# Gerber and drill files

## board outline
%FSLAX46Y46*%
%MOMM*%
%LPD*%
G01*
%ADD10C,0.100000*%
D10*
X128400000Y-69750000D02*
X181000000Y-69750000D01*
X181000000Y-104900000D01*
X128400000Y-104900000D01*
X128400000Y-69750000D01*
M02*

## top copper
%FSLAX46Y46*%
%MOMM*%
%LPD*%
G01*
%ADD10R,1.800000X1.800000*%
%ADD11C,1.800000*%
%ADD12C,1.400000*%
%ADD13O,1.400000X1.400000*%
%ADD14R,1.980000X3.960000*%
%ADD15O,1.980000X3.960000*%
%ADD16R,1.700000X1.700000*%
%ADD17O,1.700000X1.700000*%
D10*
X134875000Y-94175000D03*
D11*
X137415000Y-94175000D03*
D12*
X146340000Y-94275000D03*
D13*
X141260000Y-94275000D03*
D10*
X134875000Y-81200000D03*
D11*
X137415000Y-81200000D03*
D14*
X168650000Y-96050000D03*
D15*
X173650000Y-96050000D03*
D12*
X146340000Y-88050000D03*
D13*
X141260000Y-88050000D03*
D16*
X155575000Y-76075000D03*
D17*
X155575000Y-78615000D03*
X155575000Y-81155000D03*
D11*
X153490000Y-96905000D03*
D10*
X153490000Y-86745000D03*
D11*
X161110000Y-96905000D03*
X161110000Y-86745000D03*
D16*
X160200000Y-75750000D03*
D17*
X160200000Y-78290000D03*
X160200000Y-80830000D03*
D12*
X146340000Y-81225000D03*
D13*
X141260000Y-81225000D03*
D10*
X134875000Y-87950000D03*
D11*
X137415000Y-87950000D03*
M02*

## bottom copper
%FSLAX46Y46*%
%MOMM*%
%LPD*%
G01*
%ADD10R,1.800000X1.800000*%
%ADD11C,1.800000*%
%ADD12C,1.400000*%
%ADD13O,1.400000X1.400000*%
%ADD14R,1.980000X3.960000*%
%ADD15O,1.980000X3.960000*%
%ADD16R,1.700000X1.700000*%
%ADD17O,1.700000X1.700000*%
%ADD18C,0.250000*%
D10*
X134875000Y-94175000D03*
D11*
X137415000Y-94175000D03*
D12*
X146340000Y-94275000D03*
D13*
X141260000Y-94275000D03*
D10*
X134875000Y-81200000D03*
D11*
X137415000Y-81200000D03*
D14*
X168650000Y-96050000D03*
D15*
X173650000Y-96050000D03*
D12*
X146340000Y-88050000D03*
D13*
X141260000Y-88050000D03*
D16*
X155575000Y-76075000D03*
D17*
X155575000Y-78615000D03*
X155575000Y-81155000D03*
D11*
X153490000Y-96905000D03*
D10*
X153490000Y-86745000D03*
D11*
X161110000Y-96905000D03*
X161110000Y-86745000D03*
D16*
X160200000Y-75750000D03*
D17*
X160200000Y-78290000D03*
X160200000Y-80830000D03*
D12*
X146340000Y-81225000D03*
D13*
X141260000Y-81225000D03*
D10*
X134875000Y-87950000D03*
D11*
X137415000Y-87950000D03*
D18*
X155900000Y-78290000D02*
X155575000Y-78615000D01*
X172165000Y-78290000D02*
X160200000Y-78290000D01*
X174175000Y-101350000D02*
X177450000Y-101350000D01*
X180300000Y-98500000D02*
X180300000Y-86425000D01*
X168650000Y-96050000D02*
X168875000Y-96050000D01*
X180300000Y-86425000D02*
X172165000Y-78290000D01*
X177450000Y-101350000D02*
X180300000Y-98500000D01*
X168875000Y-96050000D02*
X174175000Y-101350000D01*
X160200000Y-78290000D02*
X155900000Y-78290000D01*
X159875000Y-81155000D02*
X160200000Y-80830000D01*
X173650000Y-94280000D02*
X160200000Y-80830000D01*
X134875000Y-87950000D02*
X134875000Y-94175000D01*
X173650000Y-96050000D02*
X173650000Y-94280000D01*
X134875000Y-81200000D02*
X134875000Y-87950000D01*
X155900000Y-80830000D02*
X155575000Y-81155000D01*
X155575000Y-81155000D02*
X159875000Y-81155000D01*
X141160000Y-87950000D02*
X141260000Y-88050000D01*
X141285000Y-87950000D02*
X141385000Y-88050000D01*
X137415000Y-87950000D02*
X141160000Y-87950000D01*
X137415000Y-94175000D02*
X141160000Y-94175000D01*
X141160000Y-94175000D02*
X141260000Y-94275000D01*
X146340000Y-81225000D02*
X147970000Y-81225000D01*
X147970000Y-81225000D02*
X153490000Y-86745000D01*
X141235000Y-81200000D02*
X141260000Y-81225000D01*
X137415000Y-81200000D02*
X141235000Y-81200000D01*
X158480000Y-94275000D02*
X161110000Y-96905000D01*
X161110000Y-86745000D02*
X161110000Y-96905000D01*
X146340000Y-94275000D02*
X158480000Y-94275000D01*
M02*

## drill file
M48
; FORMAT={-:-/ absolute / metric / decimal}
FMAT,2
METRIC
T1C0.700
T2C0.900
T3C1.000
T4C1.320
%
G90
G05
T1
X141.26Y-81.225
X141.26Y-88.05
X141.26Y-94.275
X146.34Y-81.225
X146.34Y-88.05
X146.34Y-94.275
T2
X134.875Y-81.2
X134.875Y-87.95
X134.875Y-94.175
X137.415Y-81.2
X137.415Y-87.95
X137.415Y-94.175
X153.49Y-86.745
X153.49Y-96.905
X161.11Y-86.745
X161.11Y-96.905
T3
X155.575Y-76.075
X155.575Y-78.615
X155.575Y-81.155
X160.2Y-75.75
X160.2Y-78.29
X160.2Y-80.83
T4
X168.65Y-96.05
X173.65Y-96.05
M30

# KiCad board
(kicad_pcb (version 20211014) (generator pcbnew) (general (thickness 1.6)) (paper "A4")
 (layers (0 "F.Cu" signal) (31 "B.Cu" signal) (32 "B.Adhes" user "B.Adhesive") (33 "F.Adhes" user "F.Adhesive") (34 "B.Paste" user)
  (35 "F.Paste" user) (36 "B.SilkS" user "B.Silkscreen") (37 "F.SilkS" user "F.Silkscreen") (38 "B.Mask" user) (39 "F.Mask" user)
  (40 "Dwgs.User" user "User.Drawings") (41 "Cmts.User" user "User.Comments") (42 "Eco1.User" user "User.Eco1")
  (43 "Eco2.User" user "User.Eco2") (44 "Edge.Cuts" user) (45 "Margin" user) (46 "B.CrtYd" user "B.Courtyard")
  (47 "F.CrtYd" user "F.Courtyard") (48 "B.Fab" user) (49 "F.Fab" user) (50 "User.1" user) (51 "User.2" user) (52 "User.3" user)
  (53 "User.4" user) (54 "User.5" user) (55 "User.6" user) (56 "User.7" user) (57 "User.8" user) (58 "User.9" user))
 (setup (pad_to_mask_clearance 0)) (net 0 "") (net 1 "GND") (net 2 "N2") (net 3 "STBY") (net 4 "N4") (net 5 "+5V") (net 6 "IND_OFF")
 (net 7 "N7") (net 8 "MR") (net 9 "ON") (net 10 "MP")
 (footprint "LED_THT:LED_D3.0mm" (layer "F.Cu") (at 134.875 94.175)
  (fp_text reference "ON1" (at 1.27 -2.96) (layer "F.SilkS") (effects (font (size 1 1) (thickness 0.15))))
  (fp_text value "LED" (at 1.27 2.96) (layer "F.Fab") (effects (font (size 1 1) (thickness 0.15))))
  (pad "1" thru_hole rect (at 0 0) (size 1.8 1.8) (drill 0.9) (layers *.Cu *.Mask) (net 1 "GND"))
  (pad "2" thru_hole circle (at 2.54 0) (size 1.8 1.8) (drill 0.9) (layers *.Cu *.Mask) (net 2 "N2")))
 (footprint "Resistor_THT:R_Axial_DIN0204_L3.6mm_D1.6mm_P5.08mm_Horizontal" (layer "F.Cu") (at 146.34 94.275 180)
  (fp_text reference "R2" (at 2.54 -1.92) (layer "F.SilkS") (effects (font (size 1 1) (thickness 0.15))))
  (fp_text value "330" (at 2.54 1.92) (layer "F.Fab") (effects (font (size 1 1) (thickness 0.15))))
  (pad "1" thru_hole circle (at 0 0 180) (size 1.4 1.4) (drill 0.7) (layers *.Cu *.Mask) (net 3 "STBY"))
  (pad "2" thru_hole oval (at 5.08 0 180) (size 1.4 1.4) (drill 0.7) (layers *.Cu *.Mask) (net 2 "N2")))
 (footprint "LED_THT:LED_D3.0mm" (layer "F.Cu") (at 134.875 81.2)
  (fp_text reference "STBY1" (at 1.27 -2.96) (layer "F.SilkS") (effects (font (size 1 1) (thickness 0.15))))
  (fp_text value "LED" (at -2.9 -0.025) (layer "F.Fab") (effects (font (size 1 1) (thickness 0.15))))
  (pad "1" thru_hole rect (at 0 0) (size 1.8 1.8) (drill 0.9) (layers *.Cu *.Mask) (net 1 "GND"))
  (pad "2" thru_hole circle (at 2.54 0) (size 1.8 1.8) (drill 0.9) (layers *.Cu *.Mask) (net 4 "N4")))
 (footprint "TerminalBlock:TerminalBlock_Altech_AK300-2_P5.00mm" (layer "F.Cu") (at 168.65 96.05)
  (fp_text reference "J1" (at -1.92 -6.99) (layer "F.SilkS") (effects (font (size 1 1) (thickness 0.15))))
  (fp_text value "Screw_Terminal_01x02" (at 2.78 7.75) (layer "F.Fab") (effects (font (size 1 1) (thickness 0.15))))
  (pad "1" thru_hole rect (at 0 0) (size 1.98 3.96) (drill 1.32) (layers *.Cu *.Mask) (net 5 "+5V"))
  (pad "2" thru_hole oval (at 5 0) (size 1.98 3.96) (drill 1.32) (layers *.Cu *.Mask) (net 1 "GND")))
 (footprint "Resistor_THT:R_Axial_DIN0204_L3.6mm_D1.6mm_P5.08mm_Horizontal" (layer "F.Cu") (at 146.34 88.05 180)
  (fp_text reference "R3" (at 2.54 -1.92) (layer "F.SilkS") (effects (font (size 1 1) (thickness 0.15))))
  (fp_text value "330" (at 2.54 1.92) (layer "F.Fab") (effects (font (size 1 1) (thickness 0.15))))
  (pad "1" thru_hole circle (at 0 0 180) (size 1.4 1.4) (drill 0.7) (layers *.Cu *.Mask) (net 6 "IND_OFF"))
  (pad "2" thru_hole oval (at 5.08 0 180) (size 1.4 1.4) (drill 0.7) (layers *.Cu *.Mask) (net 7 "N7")))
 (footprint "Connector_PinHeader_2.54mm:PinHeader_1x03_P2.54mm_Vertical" (layer "F.Cu") (at 155.575 76.075)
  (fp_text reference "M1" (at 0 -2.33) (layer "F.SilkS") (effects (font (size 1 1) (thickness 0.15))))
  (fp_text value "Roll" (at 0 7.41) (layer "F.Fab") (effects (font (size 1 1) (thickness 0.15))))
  (pad "1" thru_hole rect (at 0 0) (size 1.7 1.7) (drill 1) (layers *.Cu *.Mask) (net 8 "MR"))
  (pad "2" thru_hole oval (at 0 2.54) (size 1.7 1.7) (drill 1) (layers *.Cu *.Mask) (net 5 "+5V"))
  (pad "3" thru_hole oval (at 0 5.08) (size 1.7 1.7) (drill 1) (layers *.Cu *.Mask) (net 1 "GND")))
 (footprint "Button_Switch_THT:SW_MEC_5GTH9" (layer "F.Cu") (at 153.49 86.745)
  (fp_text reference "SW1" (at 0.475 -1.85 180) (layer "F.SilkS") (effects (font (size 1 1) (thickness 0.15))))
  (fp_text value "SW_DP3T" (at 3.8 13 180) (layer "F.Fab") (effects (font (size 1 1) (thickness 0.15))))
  (pad "1" thru_hole circle (at 0 10.16 90) (size 1.8 1.8) (drill 0.9) (layers *.Cu *.Mask) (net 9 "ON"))
  (pad "1" thru_hole rect (at 0 0 90) (size 1.8 1.8) (drill 0.9) (layers *.Cu *.Mask) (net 9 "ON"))
  (pad "2" thru_hole circle (at 7.62 10.16 90) (size 1.8 1.8) (drill 0.9) (layers *.Cu *.Mask) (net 3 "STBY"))
  (pad "2" thru_hole circle (at 7.62 0 90) (size 1.8 1.8) (drill 0.9) (layers *.Cu *.Mask) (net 3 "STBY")))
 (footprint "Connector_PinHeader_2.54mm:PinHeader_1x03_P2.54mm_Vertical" (layer "F.Cu") (at 160.2 75.75)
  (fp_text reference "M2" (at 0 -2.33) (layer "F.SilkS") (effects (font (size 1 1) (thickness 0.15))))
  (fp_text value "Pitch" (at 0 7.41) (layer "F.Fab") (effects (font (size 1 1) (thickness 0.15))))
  (pad "1" thru_hole rect (at 0 0) (size 1.7 1.7) (drill 1) (layers *.Cu *.Mask) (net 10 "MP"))
  (pad "2" thru_hole oval (at 0 2.54) (size 1.7 1.7) (drill 1) (layers *.Cu *.Mask) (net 5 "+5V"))
  (pad "3" thru_hole oval (at 0 5.08) (size 1.7 1.7) (drill 1) (layers *.Cu *.Mask) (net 1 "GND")))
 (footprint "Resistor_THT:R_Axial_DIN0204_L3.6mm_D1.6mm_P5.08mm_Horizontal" (layer "F.Cu") (at 146.34 81.225 180)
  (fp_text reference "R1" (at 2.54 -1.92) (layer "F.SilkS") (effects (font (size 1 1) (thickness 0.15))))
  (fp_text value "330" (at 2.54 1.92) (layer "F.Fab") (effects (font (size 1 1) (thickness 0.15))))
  (pad "1" thru_hole circle (at 0 0 180) (size 1.4 1.4) (drill 0.7) (layers *.Cu *.Mask) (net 9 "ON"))
  (pad "2" thru_hole oval (at 5.08 0 180) (size 1.4 1.4) (drill 0.7) (layers *.Cu *.Mask) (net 4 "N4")))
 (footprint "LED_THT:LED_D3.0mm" (layer "F.Cu") (at 134.875 87.95)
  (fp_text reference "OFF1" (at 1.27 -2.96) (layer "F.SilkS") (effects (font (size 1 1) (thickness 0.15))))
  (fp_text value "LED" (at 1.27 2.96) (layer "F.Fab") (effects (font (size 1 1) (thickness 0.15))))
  (pad "1" thru_hole rect (at 0 0) (size 1.8 1.8) (drill 0.9) (layers *.Cu *.Mask) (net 1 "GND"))
  (pad "2" thru_hole circle (at 2.54 0) (size 1.8 1.8) (drill 0.9) (layers *.Cu *.Mask) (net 7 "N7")))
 (gr_rect (start 128.4 104.9) (end 181 69.75) (layer "Edge.Cuts") (width 0.1) (fill none))
 (segment (start 155.9 78.29) (end 155.575 78.615) (width 0.25) (layer "B.Cu") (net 5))
 (segment (start 172.165 78.29) (end 160.2 78.29) (width 0.25) (layer "B.Cu") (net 5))
 (segment (start 174.175 101.35) (end 177.45 101.35) (width 0.25) (layer "B.Cu") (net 5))
 (segment (start 180.3 98.5) (end 180.3 86.425) (width 0.25) (layer "B.Cu") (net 5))
 (segment (start 168.65 96.05) (end 168.875 96.05) (width 0.25) (layer "B.Cu") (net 5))
 (segment (start 180.3 86.425) (end 172.165 78.29) (width 0.25) (layer "B.Cu") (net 5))
 (segment (start 177.45 101.35) (end 180.3 98.5) (width 0.25) (layer "B.Cu") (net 5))
 (segment (start 168.875 96.05) (end 174.175 101.35) (width 0.25) (layer "B.Cu") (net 5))
 (segment (start 160.2 78.29) (end 155.9 78.29) (width 0.25) (layer "B.Cu") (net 5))
 (segment (start 159.875 81.155) (end 160.2 80.83) (width 0.25) (layer "B.Cu") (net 1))
 (segment (start 173.65 94.28) (end 160.2 80.83) (width 0.25) (layer "B.Cu") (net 1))
 (segment (start 134.875 87.95) (end 134.875 94.175) (width 0.25) (layer "B.Cu") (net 1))
 (segment (start 173.65 96.05) (end 173.65 94.28) (width 0.25) (layer "B.Cu") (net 1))
 (segment (start 134.875 81.2) (end 134.875 87.95) (width 0.25) (layer "B.Cu") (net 1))
 (segment (start 155.9 80.83) (end 155.575 81.155) (width 0.25) (layer "B.Cu") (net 1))
 (segment (start 155.575 81.155) (end 159.875 81.155) (width 0.25) (layer "B.Cu") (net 1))
 (segment (start 141.16 87.95) (end 141.26 88.05) (width 0.25) (layer "B.Cu") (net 7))
 (segment (start 141.285 87.95) (end 141.385 88.05) (width 0.25) (layer "B.Cu") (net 7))
 (segment (start 137.415 87.95) (end 141.16 87.95) (width 0.25) (layer "B.Cu") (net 7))
 (segment (start 137.415 94.175) (end 141.16 94.175) (width 0.25) (layer "B.Cu") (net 2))
 (segment (start 141.16 94.175) (end 141.26 94.275) (width 0.25) (layer "B.Cu") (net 2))
 (segment (start 146.34 81.225) (end 147.97 81.225) (width 0.25) (layer "B.Cu") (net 9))
 (segment (start 147.97 81.225) (end 153.49 86.745) (width 0.25) (layer "B.Cu") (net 9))
 (segment (start 141.235 81.2) (end 141.26 81.225) (width 0.25) (layer "B.Cu") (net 4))
 (segment (start 137.415 81.2) (end 141.235 81.2) (width 0.25) (layer "B.Cu") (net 4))
 (segment (start 158.48 94.275) (end 161.11 96.905) (width 0.25) (layer "B.Cu") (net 3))
 (segment (start 161.11 86.745) (end 161.11 96.905) (width 0.25) (layer "B.Cu") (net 3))
 (segment (start 146.34 94.275) (end 158.48 94.275) (width 0.25) (layer "B.Cu") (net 3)))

